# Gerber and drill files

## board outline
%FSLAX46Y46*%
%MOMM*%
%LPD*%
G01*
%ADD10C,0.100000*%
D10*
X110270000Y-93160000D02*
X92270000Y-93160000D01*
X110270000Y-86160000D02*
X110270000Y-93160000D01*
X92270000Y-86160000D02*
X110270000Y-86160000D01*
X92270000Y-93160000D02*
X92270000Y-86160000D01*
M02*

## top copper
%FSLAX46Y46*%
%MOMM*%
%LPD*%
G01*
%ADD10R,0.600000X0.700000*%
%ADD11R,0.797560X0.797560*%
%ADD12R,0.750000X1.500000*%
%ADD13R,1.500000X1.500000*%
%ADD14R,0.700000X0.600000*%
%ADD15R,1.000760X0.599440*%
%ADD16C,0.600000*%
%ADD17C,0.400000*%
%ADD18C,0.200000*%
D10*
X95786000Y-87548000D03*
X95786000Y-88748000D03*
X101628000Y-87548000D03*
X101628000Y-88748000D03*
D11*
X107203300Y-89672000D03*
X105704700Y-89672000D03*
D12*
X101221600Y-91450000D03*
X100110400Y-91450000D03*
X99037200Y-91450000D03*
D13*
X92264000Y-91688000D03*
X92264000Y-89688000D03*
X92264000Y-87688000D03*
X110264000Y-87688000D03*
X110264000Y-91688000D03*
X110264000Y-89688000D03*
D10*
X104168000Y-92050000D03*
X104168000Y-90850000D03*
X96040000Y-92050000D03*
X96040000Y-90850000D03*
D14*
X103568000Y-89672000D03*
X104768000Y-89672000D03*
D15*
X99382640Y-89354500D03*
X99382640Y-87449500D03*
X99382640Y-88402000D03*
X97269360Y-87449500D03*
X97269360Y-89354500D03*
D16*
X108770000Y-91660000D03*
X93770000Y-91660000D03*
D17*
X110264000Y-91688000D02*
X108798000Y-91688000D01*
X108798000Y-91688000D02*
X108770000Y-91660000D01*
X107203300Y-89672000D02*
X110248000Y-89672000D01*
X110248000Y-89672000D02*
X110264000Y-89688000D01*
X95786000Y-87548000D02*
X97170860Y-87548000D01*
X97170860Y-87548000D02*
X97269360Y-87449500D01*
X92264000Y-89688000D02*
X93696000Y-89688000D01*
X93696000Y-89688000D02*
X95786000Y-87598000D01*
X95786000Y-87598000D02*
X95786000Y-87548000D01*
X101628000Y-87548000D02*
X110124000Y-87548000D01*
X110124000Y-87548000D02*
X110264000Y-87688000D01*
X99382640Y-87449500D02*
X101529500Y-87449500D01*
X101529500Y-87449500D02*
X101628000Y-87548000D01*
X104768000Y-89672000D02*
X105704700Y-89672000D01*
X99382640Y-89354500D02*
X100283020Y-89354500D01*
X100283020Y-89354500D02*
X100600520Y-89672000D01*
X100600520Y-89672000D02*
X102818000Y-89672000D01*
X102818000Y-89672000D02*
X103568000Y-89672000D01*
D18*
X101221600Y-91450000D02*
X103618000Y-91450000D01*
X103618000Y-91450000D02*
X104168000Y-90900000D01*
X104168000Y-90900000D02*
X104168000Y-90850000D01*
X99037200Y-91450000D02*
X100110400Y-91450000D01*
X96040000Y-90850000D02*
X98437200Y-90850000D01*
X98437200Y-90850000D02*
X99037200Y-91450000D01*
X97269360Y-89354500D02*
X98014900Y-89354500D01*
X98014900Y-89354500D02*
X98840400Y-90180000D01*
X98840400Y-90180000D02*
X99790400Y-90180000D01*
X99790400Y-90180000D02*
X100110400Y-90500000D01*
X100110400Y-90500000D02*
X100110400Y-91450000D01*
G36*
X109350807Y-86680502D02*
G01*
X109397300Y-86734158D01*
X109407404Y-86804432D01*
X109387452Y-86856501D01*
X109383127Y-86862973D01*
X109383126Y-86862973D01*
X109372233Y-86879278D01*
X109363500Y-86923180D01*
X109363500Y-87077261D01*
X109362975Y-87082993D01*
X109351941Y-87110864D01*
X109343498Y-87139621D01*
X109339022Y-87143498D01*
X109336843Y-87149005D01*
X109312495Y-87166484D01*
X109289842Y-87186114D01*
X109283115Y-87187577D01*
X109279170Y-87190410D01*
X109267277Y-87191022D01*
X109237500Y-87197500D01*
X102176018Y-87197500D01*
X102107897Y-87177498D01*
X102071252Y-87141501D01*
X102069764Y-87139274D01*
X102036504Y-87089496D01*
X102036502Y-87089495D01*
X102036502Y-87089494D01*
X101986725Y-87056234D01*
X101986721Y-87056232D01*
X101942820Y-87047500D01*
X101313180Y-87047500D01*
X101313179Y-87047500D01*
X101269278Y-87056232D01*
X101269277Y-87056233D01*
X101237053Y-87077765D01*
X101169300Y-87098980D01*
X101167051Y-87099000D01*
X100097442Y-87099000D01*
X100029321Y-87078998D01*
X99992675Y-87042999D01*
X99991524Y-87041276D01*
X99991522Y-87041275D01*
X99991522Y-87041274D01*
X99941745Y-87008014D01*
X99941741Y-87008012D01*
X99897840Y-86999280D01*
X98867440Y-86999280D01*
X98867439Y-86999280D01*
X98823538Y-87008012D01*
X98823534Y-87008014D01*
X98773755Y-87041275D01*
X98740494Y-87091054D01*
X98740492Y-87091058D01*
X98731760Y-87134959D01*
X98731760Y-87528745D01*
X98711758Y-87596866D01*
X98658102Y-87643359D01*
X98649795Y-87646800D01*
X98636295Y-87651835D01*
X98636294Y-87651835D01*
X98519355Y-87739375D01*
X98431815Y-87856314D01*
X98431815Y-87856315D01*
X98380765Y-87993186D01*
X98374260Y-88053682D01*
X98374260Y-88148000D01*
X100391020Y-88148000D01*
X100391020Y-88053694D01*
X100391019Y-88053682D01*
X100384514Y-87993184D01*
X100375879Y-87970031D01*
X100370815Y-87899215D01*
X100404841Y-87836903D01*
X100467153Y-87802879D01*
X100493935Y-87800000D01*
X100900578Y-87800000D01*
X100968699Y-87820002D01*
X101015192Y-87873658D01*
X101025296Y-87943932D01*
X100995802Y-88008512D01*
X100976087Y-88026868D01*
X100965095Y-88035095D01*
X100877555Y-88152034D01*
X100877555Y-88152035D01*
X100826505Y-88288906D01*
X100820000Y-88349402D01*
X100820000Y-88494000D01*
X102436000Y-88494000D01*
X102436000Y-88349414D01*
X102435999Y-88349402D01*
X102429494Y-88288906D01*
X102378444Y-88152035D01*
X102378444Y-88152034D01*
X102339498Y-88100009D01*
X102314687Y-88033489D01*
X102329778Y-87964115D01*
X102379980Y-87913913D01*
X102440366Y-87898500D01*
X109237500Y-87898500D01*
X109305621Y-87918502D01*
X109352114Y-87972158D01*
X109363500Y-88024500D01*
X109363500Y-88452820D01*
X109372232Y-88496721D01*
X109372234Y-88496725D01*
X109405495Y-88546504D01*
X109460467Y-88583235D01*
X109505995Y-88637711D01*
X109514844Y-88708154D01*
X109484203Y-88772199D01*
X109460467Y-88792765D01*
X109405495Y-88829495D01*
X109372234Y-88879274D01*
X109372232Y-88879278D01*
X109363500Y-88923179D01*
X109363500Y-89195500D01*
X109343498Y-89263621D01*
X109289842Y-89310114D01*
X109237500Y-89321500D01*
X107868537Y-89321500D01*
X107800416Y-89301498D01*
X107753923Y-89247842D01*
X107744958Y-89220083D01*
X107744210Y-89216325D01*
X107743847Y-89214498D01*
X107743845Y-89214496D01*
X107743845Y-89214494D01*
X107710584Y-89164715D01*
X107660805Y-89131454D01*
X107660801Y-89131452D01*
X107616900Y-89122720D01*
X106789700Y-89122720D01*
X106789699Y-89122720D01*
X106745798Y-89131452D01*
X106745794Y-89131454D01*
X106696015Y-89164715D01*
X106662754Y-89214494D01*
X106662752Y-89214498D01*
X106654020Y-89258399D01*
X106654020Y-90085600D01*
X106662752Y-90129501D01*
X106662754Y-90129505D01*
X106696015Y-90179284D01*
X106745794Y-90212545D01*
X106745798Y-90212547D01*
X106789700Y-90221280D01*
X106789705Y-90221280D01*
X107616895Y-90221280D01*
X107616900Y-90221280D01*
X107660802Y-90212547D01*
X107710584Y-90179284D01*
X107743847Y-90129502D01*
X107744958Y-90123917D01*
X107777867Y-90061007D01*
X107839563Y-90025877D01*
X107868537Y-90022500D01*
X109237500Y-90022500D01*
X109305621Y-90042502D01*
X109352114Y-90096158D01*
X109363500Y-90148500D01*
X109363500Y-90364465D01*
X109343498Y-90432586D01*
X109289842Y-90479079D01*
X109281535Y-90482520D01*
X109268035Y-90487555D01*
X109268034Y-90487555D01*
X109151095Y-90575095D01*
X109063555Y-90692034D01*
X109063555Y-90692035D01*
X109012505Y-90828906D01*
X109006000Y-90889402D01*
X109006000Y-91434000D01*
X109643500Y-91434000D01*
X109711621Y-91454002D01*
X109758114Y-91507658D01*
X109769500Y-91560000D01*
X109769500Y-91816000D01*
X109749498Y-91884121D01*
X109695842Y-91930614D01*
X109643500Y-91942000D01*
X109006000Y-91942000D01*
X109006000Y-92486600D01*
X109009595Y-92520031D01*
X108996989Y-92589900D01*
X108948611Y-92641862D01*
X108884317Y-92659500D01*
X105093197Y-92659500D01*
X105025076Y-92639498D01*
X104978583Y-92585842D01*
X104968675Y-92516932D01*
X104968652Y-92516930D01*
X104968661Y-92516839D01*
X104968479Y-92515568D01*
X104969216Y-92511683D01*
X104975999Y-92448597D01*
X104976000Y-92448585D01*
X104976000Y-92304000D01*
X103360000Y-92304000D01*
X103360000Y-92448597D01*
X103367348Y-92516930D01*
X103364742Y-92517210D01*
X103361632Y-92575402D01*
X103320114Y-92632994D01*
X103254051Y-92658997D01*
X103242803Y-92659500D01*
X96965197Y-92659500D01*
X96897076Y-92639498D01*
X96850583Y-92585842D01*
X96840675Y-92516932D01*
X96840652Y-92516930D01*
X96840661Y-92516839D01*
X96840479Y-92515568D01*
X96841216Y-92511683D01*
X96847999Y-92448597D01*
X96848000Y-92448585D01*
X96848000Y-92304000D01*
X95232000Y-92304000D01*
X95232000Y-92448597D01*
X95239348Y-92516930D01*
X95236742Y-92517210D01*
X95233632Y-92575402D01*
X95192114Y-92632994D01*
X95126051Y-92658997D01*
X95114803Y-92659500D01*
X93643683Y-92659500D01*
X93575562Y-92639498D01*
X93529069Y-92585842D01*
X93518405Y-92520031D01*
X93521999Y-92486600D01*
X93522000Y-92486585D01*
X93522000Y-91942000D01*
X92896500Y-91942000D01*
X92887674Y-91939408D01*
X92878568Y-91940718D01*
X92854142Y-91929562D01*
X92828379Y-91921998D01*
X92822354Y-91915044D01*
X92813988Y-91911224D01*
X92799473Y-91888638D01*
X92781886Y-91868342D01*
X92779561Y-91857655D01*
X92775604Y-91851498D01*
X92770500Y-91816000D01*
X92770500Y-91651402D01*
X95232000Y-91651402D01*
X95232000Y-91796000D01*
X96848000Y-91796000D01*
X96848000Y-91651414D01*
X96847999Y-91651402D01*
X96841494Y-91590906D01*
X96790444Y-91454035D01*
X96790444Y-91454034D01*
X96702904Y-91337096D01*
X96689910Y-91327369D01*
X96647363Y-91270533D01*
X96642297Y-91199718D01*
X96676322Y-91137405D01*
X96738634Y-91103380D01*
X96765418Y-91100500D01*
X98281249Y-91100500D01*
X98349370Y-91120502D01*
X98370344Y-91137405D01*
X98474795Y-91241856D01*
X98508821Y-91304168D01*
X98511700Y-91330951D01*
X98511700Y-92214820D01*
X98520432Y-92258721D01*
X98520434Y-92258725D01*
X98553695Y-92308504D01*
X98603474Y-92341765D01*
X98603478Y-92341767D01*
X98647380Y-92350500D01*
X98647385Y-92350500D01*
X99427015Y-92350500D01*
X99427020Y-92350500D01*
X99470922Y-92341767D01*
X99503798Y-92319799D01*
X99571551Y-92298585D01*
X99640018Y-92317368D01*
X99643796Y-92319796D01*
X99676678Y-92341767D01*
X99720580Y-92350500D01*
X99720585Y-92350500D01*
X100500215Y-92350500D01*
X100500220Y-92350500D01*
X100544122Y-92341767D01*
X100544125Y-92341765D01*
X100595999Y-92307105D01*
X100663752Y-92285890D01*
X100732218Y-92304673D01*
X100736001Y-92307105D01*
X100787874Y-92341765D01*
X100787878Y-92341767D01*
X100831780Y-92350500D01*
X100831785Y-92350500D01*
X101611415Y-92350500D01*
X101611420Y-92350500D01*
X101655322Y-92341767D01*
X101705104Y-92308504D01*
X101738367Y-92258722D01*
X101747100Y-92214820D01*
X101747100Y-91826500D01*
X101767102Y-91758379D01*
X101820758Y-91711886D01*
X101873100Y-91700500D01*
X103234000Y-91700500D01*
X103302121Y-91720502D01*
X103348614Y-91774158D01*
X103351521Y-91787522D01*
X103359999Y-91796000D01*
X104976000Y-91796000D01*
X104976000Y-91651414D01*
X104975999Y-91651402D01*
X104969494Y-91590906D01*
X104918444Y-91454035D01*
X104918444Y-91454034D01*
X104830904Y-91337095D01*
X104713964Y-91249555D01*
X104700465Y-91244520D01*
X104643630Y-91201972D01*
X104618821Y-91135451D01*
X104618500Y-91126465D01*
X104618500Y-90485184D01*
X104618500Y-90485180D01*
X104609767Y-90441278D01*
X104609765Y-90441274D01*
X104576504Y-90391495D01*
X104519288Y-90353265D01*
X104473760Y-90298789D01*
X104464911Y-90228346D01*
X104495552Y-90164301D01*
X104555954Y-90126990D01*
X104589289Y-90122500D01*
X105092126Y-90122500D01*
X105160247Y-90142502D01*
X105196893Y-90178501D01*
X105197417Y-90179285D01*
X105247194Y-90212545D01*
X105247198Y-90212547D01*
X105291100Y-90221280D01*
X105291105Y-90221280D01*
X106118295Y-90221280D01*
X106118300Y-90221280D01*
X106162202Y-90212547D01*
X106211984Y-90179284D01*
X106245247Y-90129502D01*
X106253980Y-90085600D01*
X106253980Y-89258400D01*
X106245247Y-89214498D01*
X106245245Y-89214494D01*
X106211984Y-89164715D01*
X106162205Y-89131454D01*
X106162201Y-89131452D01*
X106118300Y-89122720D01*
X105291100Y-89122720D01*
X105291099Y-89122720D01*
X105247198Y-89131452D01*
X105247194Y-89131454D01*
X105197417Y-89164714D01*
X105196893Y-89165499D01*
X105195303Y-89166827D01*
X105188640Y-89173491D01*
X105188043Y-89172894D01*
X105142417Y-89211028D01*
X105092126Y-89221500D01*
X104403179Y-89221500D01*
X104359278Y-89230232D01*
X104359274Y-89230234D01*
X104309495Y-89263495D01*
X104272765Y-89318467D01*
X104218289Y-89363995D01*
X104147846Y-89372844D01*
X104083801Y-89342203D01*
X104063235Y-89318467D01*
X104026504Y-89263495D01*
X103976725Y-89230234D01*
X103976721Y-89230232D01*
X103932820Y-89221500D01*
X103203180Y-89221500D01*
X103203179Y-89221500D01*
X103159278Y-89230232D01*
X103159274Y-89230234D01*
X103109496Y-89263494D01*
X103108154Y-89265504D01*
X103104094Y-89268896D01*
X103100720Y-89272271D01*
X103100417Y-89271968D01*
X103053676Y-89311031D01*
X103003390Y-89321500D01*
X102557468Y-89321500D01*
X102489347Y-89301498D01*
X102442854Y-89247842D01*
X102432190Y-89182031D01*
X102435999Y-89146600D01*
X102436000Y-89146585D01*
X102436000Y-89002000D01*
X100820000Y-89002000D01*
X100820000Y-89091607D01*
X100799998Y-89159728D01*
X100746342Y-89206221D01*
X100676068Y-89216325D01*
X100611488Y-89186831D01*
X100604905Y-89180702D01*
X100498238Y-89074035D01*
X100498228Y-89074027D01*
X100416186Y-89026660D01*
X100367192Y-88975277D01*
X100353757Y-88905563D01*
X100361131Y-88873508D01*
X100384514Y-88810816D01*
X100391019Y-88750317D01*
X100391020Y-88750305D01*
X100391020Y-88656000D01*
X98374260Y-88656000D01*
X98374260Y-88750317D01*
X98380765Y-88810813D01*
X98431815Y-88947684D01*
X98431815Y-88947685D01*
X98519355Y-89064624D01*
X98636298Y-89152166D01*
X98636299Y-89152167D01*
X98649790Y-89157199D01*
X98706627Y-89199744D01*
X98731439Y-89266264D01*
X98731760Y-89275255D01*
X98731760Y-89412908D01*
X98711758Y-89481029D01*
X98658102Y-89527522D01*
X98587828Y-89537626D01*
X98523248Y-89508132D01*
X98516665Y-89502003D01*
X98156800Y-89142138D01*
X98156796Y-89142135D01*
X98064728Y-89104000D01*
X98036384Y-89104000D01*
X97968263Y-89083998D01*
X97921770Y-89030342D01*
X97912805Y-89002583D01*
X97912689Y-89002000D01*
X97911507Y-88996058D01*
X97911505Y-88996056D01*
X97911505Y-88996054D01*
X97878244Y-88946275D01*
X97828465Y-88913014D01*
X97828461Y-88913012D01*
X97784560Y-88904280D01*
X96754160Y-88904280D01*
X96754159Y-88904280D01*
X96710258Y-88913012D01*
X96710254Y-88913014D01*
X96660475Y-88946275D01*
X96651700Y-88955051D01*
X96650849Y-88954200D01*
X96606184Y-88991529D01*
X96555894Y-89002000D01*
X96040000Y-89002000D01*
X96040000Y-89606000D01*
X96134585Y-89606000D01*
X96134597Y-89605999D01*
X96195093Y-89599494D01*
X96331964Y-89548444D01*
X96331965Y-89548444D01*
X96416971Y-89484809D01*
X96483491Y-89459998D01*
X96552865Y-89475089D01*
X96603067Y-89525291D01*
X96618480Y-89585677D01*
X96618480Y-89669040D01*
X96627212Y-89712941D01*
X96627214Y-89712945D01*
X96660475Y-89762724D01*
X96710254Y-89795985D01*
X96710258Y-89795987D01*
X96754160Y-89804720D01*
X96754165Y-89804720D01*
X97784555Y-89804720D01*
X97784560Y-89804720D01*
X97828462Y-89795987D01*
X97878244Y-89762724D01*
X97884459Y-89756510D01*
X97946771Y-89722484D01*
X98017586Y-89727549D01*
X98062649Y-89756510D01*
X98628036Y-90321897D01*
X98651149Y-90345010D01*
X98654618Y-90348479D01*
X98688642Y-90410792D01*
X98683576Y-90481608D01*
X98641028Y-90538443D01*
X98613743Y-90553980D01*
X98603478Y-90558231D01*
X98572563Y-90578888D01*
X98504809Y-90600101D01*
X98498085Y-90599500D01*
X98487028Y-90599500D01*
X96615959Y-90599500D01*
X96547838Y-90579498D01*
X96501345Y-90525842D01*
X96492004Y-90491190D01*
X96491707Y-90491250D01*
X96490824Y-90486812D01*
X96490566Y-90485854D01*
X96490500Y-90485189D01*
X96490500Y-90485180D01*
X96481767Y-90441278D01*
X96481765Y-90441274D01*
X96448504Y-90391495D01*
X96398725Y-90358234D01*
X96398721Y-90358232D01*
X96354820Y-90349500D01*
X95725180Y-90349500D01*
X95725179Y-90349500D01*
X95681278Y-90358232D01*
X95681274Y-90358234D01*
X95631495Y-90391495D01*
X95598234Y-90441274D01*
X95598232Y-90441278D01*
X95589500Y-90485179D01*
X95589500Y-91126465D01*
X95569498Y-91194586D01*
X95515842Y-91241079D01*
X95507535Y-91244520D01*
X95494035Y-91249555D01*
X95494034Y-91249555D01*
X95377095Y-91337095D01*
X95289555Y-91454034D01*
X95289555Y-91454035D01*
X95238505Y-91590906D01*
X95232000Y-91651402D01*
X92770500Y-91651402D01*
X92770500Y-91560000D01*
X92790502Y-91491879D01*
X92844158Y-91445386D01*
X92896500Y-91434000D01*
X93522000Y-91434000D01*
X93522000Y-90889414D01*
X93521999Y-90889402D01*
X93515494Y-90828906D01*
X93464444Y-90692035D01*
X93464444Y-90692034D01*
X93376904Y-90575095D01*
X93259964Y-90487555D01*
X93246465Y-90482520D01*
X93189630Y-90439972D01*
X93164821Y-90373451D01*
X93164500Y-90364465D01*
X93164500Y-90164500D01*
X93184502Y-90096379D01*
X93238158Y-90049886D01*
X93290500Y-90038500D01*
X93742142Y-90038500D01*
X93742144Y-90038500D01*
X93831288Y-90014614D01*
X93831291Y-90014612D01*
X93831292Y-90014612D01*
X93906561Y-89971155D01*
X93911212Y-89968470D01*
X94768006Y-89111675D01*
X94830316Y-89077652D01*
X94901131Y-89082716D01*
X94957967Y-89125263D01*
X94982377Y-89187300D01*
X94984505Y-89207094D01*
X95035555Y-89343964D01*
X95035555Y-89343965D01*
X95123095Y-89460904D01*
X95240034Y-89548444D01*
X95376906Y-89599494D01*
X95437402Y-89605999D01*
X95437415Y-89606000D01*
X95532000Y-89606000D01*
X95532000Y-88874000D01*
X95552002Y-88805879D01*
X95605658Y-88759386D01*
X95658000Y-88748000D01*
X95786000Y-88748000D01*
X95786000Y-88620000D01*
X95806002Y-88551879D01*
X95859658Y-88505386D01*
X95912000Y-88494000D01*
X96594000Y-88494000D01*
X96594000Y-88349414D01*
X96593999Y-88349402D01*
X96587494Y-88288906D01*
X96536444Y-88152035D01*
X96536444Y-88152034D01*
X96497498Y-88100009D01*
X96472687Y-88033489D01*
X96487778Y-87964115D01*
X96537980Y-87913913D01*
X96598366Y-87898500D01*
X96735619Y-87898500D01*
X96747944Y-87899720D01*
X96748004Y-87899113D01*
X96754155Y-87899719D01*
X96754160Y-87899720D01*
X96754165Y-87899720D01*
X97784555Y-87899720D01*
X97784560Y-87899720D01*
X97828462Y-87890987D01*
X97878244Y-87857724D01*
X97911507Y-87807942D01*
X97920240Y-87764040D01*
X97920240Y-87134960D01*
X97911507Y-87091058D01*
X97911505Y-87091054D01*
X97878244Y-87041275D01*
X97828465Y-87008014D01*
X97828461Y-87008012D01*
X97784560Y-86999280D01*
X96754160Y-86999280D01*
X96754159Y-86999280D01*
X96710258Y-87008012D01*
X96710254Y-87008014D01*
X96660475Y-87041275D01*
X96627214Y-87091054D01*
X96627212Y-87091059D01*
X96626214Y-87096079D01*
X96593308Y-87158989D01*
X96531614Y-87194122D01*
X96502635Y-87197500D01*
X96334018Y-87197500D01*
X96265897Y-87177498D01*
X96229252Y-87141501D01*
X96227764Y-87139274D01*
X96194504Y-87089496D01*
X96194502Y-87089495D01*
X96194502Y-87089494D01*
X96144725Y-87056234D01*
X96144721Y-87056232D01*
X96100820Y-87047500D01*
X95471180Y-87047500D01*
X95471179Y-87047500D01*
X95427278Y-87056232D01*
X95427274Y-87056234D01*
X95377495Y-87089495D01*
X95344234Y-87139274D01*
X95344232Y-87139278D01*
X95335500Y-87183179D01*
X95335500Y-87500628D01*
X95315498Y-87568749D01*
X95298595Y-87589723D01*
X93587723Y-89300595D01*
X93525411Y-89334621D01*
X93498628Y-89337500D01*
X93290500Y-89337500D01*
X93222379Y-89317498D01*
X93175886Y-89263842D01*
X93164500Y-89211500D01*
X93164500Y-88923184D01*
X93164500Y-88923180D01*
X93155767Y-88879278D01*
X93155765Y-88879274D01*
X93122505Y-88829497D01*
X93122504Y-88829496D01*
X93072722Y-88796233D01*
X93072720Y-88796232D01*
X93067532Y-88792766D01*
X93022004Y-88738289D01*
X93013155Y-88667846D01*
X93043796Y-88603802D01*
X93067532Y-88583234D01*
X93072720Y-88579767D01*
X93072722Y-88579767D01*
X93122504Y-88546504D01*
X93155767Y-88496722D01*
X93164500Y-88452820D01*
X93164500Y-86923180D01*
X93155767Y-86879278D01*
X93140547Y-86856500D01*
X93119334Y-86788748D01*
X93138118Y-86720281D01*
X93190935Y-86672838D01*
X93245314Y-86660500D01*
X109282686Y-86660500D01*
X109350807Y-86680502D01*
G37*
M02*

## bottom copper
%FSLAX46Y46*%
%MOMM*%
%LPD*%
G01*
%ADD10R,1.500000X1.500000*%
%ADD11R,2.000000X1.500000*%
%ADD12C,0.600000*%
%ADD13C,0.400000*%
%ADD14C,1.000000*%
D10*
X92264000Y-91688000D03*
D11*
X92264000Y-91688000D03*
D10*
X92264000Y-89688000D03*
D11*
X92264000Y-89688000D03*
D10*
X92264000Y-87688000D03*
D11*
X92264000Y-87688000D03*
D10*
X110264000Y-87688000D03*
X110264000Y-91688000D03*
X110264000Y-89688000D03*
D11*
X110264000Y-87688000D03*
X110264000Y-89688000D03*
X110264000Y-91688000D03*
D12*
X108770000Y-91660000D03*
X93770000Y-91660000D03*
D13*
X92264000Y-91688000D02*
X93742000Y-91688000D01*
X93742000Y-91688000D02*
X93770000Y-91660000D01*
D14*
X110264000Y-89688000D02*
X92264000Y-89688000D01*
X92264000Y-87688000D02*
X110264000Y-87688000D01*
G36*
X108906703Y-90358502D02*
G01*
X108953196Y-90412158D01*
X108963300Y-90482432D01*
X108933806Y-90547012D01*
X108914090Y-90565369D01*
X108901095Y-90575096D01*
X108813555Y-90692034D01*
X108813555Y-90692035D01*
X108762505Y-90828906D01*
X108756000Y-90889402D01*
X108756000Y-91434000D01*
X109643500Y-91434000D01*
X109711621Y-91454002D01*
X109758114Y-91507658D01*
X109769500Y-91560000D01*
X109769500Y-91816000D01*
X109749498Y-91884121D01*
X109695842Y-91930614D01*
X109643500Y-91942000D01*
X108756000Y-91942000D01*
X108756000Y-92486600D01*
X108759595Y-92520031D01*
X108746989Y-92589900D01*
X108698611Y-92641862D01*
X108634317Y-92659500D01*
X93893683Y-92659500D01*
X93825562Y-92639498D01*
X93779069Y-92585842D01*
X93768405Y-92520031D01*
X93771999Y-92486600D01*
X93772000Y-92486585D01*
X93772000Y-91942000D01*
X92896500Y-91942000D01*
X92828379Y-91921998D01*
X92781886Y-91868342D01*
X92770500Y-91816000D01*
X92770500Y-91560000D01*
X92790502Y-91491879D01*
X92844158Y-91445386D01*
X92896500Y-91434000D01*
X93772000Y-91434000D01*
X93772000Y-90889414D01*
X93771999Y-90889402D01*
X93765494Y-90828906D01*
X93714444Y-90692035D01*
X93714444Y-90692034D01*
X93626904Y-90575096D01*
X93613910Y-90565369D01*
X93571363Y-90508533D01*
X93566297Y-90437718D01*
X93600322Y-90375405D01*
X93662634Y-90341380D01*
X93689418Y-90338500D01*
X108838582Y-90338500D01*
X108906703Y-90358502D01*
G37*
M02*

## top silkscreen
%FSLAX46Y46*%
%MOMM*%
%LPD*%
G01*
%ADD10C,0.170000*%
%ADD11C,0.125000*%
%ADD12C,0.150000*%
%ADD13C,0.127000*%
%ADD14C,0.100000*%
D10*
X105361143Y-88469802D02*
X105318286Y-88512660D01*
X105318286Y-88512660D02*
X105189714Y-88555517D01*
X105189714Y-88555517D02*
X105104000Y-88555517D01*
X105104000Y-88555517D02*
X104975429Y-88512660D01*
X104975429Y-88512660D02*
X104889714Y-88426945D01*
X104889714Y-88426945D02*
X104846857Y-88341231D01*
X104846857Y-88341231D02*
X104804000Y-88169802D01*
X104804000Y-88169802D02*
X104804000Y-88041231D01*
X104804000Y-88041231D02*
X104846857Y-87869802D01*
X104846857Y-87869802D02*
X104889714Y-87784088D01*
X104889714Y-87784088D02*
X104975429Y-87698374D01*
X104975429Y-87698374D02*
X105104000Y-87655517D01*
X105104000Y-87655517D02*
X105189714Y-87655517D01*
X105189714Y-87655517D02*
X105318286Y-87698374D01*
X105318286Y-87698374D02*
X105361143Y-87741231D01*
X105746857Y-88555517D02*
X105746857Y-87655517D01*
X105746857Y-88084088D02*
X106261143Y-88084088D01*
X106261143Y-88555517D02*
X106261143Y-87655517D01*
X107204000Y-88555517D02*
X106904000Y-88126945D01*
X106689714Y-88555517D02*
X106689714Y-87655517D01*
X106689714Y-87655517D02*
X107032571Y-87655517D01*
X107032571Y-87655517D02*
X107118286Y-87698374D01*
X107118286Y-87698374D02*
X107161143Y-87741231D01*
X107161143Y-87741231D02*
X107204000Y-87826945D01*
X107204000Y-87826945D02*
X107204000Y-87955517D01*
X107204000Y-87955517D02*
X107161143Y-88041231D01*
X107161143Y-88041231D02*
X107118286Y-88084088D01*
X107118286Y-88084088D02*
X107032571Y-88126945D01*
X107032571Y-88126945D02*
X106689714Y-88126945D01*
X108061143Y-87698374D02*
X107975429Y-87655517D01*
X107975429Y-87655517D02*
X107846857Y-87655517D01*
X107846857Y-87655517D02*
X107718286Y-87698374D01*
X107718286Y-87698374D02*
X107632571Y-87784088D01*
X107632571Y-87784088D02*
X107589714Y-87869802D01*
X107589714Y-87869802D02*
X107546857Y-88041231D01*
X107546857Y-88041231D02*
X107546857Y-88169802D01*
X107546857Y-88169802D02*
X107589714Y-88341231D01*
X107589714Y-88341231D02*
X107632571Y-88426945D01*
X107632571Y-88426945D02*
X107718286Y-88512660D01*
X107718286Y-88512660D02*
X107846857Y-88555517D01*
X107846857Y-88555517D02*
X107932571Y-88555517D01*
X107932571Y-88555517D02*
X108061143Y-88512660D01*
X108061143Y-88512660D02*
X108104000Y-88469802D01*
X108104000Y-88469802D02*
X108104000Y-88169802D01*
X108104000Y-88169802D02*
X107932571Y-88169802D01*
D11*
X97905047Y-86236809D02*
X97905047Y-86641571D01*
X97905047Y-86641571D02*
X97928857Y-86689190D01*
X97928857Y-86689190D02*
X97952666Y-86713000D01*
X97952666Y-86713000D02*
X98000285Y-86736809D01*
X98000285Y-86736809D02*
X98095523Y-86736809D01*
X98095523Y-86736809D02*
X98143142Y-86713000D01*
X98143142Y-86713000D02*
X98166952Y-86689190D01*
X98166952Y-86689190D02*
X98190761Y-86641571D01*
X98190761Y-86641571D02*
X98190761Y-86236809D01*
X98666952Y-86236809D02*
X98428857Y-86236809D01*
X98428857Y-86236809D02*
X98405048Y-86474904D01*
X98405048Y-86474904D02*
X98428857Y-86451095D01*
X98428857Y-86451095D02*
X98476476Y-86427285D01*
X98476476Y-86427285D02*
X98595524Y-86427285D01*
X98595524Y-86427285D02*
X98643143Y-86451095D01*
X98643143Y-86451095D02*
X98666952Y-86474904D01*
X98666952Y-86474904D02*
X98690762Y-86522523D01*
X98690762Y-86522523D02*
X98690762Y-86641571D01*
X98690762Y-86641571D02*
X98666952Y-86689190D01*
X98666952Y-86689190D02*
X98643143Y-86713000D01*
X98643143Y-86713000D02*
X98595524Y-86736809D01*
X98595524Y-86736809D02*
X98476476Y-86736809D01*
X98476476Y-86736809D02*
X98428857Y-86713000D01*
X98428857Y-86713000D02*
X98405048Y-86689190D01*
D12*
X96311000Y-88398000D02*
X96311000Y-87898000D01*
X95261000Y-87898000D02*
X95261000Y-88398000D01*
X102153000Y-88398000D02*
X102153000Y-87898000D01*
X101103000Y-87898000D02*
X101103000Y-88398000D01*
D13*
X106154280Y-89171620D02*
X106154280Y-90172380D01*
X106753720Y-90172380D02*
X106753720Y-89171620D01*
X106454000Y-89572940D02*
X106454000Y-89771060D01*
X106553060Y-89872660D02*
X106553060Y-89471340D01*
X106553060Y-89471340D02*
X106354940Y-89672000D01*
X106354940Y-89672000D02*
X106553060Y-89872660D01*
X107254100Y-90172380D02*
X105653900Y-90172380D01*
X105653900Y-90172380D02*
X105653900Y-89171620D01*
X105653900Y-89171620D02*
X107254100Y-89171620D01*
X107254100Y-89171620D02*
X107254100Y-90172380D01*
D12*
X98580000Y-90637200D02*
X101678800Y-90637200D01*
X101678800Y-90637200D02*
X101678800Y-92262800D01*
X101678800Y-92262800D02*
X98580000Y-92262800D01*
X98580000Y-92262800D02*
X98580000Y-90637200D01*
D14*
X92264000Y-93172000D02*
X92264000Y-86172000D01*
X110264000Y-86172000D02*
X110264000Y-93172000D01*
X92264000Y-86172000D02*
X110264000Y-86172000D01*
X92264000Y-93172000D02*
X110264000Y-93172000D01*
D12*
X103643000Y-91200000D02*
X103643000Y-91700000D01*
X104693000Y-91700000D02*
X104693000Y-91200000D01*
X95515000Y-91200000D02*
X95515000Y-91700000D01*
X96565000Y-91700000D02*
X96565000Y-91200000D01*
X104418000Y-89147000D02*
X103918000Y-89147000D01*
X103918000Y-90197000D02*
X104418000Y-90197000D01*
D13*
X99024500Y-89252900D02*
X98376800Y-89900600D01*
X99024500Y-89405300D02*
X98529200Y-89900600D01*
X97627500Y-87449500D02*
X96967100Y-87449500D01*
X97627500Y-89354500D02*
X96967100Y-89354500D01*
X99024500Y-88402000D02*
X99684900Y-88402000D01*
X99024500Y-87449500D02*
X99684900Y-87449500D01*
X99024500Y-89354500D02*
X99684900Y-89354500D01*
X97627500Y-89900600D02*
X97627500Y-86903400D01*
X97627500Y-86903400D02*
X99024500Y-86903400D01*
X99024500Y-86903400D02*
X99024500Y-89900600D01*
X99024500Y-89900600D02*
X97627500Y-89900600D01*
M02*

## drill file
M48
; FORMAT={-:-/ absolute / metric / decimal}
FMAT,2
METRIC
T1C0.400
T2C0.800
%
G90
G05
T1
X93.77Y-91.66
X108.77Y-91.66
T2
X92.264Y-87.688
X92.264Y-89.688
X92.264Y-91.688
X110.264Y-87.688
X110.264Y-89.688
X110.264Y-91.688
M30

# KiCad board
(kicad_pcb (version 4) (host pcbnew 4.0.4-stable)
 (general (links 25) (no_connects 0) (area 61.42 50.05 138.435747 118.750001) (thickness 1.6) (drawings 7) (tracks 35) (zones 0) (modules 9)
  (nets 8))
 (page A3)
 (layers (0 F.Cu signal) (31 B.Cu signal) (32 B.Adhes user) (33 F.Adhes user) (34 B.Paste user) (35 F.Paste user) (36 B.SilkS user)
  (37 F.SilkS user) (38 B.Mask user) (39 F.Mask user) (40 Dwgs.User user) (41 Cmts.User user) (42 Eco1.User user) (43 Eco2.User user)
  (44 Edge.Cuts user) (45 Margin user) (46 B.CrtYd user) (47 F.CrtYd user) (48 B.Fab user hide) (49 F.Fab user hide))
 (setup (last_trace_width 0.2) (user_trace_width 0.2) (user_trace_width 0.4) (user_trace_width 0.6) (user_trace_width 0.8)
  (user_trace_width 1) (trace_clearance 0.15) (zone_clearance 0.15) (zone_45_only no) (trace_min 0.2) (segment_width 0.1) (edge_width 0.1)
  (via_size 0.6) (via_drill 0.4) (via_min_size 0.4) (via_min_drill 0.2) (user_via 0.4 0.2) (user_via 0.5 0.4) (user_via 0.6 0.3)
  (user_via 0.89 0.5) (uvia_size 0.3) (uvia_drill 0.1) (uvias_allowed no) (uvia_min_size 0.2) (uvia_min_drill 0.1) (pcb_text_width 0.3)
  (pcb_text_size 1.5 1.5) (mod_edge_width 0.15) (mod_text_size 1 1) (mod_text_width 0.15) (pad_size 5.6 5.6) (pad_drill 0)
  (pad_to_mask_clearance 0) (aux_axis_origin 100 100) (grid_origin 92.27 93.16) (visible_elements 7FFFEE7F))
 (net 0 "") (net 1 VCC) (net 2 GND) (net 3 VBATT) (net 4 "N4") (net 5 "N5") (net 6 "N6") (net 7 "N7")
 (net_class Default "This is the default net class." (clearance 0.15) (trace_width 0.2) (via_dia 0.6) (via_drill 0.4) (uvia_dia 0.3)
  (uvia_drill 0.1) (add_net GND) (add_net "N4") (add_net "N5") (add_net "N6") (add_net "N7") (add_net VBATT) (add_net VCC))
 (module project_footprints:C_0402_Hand (layer F.Cu) (at 95.786 88.148 270)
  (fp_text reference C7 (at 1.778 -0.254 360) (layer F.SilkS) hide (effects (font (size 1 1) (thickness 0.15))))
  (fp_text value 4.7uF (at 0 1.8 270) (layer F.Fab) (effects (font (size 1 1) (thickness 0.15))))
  (fp_line (start 0.25 -0.525) (end -0.25 -0.525) (layer F.SilkS) (width 0.15))
  (fp_line (start -0.25 0.525) (end 0.25 0.525) (layer F.SilkS) (width 0.15))
  (pad 1 smd rect (at -0.6 0 270) (size 0.7 0.6) (layers F.Cu F.Paste F.Mask) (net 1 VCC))
  (pad 2 smd rect (at 0.6 0 270) (size 0.7 0.6) (layers F.Cu F.Paste F.Mask) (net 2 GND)))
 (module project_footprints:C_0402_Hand (layer F.Cu) (at 101.628 88.148 270)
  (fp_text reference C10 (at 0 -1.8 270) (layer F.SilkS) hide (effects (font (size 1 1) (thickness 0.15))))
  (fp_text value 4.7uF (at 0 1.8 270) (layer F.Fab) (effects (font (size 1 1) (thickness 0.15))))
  (fp_line (start 0.25 -0.525) (end -0.25 -0.525) (layer F.SilkS) (width 0.15))
  (fp_line (start -0.25 0.525) (end 0.25 0.525) (layer F.SilkS) (width 0.15))
  (pad 1 smd rect (at -0.6 0 270) (size 0.7 0.6) (layers F.Cu F.Paste F.Mask) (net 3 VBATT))
  (pad 2 smd rect (at 0.6 0 270) (size 0.7 0.6) (layers F.Cu F.Paste F.Mask) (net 2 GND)))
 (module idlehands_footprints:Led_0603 (layer F.Cu) (at 106.454 89.672 180)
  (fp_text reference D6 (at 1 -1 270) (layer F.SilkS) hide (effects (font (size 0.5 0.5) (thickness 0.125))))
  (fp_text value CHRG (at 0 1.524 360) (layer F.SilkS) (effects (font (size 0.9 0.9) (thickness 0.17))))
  (fp_line (start 0.29972 0.50038) (end 0.29972 -0.50038) (layer F.SilkS) (width 0.127))
  (fp_line (start -0.29972 -0.50038) (end -0.29972 0.50038) (layer F.SilkS) (width 0.127))
  (fp_line (start 0 0.09906) (end 0 -0.09906) (layer F.SilkS) (width 0.127))
  (fp_line (start -0.09906 -0.20066) (end -0.09906 0.20066) (layer F.SilkS) (width 0.127))
  (fp_line (start -0.09906 0.20066) (end 0.09906 0) (layer F.SilkS) (width 0.127))
  (fp_line (start 0.09906 0) (end -0.09906 -0.20066) (layer F.SilkS) (width 0.127))
  (fp_line (start -0.8001 -0.50038) (end 0.8001 -0.50038) (layer F.SilkS) (width 0.127))
  (fp_line (start 0.8001 -0.50038) (end 0.8001 0.50038) (layer F.SilkS) (width 0.127))
  (fp_line (start 0.8001 0.50038) (end -0.8001 0.50038) (layer F.SilkS) (width 0.127))
  (fp_line (start -0.8001 0.50038) (end -0.8001 -0.50038) (layer F.SilkS) (width 0.127))
  (pad 2 smd rect (at -0.7493 0 180) (size 0.79756 0.79756) (layers F.Cu F.Paste F.Mask) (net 1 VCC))
  (pad 1 smd rect (at 0.7493 0 180) (size 0.79756 0.79756) (layers F.Cu F.Paste F.Mask) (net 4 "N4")))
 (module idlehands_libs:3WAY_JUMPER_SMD (layer F.Cu) (at 100.104 91.45)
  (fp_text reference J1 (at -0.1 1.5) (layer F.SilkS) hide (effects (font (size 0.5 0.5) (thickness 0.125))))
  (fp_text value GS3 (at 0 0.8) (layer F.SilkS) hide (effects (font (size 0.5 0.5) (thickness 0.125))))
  (fp_line (start -1.524 -0.8128) (end 1.5748 -0.8128) (layer F.SilkS) (width 0.15))
  (fp_line (start 1.5748 -0.8128) (end 1.5748 0.8128) (layer F.SilkS) (width 0.15))
  (fp_line (start 1.5748 0.8128) (end -1.524 0.8128) (layer F.SilkS) (width 0.15))
  (fp_line (start -1.524 0.8128) (end -1.524 -0.8128) (layer F.SilkS) (width 0.15))
  (pad 1 smd rect (at 1.1176 0) (size 0.75 1.5) (layers F.Cu F.Paste F.Mask) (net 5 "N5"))
  (pad 2 smd rect (at 0.0064 0) (size 0.75 1.5) (layers F.Cu F.Paste F.Mask) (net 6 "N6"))
  (pad 3 smd rect (at -1.0668 0) (size 0.75 1.5) (layers F.Cu F.Paste F.Mask) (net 6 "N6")))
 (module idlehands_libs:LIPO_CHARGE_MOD (layer F.Cu) (at 101.264 89.672)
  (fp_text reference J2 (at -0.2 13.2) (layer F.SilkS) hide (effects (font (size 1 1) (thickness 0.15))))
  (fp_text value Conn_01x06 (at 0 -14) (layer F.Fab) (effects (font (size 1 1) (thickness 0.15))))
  (fp_line (start -9 3.5) (end -9 -3.5) (layer F.SilkS) (width 0.1))
  (fp_line (start 9 -3.5) (end 9 3.5) (layer F.SilkS) (width 0.1))
  (fp_line (start -9 -3.5) (end 9 -3.5) (layer F.SilkS) (width 0.1))
  (fp_line (start -9 3.5) (end 9 3.5) (layer F.SilkS) (width 0.1))
  (pad 3 thru_hole rect (at -9 2.016) (size 1.5 1.5) (drill 0.8) (layers *.Cu *.Mask) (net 2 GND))
  (pad 3 smd rect (at -9 2.016) (size 2 1.5) (layers B.Cu B.Mask) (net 2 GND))
  (pad 2 thru_hole rect (at -9 0.016) (size 1.5 1.5) (drill 0.8) (layers *.Cu *.Mask) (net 1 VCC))
  (pad 2 smd rect (at -9 0.016) (size 2 1.5) (layers B.Cu B.Mask) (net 1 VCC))
  (pad 1 thru_hole rect (at -9 -1.984) (size 1.5 1.5) (drill 0.8) (layers *.Cu *.Mask) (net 3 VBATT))
  (pad 1 smd rect (at -9 -1.984) (size 2 1.5) (layers B.Cu B.Mask) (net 3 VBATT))
  (pad 4 thru_hole rect (at 9 -1.984) (size 1.5 1.5) (drill 0.8) (layers *.Cu *.Mask) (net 3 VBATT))
  (pad 6 thru_hole rect (at 9 2.016) (size 1.5 1.5) (drill 0.8) (layers *.Cu *.Mask) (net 2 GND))
  (pad 5 thru_hole rect (at 9 0.016) (size 1.5 1.5) (drill 0.8) (layers *.Cu *.Mask) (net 1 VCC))
  (pad 4 smd rect (at 9 -1.984) (size 2 1.5) (layers B.Cu B.Mask) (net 3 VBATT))
  (pad 5 smd rect (at 9 0.016) (size 2 1.5) (layers B.Cu B.Mask) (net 1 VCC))
  (pad 6 smd rect (at 9 2.016) (size 2 1.5) (layers B.Cu B.Mask) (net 2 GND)))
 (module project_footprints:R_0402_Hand (layer F.Cu) (at 104.168 91.45 90)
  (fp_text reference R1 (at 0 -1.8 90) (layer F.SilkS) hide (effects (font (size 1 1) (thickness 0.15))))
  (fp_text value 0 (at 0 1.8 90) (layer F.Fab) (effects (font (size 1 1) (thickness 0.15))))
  (fp_line (start 0.25 -0.525) (end -0.25 -0.525) (layer F.SilkS) (width 0.15))
  (fp_line (start -0.25 0.525) (end 0.25 0.525) (layer F.SilkS) (width 0.15))
  (pad 1 smd rect (at -0.6 0 90) (size 0.7 0.6) (layers F.Cu F.Paste F.Mask) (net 2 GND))
  (pad 2 smd rect (at 0.6 0 90) (size 0.7 0.6) (layers F.Cu F.Paste F.Mask) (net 5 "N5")))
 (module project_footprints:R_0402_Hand (layer F.Cu) (at 96.04 91.45 90)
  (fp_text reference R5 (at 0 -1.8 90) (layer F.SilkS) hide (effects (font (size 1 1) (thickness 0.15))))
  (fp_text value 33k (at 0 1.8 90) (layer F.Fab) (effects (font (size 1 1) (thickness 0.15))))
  (fp_line (start 0.25 -0.525) (end -0.25 -0.525) (layer F.SilkS) (width 0.15))
  (fp_line (start -0.25 0.525) (end 0.25 0.525) (layer F.SilkS) (width 0.15))
  (pad 1 smd rect (at -0.6 0 90) (size 0.7 0.6) (layers F.Cu F.Paste F.Mask) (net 2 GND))
  (pad 2 smd rect (at 0.6 0 90) (size 0.7 0.6) (layers F.Cu F.Paste F.Mask) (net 6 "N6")))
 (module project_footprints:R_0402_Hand (layer F.Cu) (at 104.168 89.672)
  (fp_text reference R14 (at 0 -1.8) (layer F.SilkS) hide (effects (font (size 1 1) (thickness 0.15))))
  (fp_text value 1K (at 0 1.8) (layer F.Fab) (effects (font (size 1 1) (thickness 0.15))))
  (fp_line (start 0.25 -0.525) (end -0.25 -0.525) (layer F.SilkS) (width 0.15))
  (fp_line (start -0.25 0.525) (end 0.25 0.525) (layer F.SilkS) (width 0.15))
  (pad 1 smd rect (at -0.6 0) (size 0.7 0.6) (layers F.Cu F.Paste F.Mask) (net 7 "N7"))
  (pad 2 smd rect (at 0.6 0) (size 0.7 0.6) (layers F.Cu F.Paste F.Mask) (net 4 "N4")))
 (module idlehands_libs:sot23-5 (layer F.Cu) (at 98.326 88.402 90)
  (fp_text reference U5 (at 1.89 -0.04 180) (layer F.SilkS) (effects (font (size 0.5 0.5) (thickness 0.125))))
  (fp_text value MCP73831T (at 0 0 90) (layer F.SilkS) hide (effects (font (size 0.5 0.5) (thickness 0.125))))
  (fp_line (start -0.8509 0.6985) (end -1.4986 0.0508) (layer F.SilkS) (width 0.127))
  (fp_line (start -1.0033 0.6985) (end -1.4986 0.2032) (layer F.SilkS) (width 0.127))
  (fp_line (start 0.9525 -0.6985) (end 0.9525 -1.3589) (layer F.SilkS) (width 0.127))
  (fp_line (start -0.9525 -0.6985) (end -0.9525 -1.3589) (layer F.SilkS) (width 0.127))
  (fp_line (start 0 0.6985) (end 0 1.3589) (layer F.SilkS) (width 0.127))
  (fp_line (start 0.9525 0.6985) (end 0.9525 1.3589) (layer F.SilkS) (width 0.127))
  (fp_line (start -0.9525 0.6985) (end -0.9525 1.3589) (layer F.SilkS) (width 0.127))
  (fp_line (start -1.4986 -0.6985) (end 1.4986 -0.6985) (layer F.SilkS) (width 0.127))
  (fp_line (start 1.4986 -0.6985) (end 1.4986 0.6985) (layer F.SilkS) (width 0.127))
  (fp_line (start 1.4986 0.6985) (end -1.4986 0.6985) (layer F.SilkS) (width 0.127))
  (fp_line (start -1.4986 0.6985) (end -1.4986 -0.6985) (layer F.SilkS) (width 0.127))
  (pad 1 smd rect (at -0.9525 1.05664 90) (size 0.59944 1.00076) (layers F.Cu F.Paste F.Mask) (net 7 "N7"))
  (pad 3 smd rect (at 0.9525 1.05664 90) (size 0.59944 1.00076) (layers F.Cu F.Paste F.Mask) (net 3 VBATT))
  (pad 2 smd rect (at 0 1.05664 90) (size 0.59944 1.00076) (layers F.Cu F.Paste F.Mask) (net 2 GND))
  (pad 4 smd rect (at 0.9525 -1.05664 90) (size 0.59944 1.00076) (layers F.Cu F.Paste F.Mask) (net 1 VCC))
  (pad 5 smd rect (at -0.9525 -1.05664 90) (size 0.59944 1.00076) (layers F.Cu F.Paste F.Mask) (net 6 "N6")))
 (gr_line (start 110.27 93.16) (end 92.27 93.16) (layer Edge.Cuts) (width 0.1))
 (gr_line (start 110.27 86.16) (end 110.27 93.16) (layer Edge.Cuts) (width 0.1))
 (gr_line (start 92.27 86.16) (end 110.27 86.16) (layer Edge.Cuts) (width 0.1))
 (gr_line (start 92.27 93.16) (end 92.27 86.16) (layer Edge.Cuts) (width 0.1))
 (segment (start 110.264 91.688) (end 108.798 91.688) (width 0.4) (layer F.Cu) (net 2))
 (segment (start 108.798 91.688) (end 108.77 91.66) (width 0.4) (layer F.Cu) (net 2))
 (via (at 108.77 91.66) (size 0.6) (drill 0.4) (layers F.Cu B.Cu) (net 2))
 (segment (start 92.264 91.688) (end 93.742 91.688) (width 0.4) (layer B.Cu) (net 2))
 (segment (start 93.742 91.688) (end 93.77 91.66) (width 0.4) (layer B.Cu) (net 2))
 (via (at 93.77 91.66) (size 0.6) (drill 0.4) (layers F.Cu B.Cu) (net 2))
 (segment (start 110.264 89.688) (end 92.264 89.688) (width 1) (layer B.Cu) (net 1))
 (segment (start 107.2033 89.672) (end 110.248 89.672) (width 0.4) (layer F.Cu) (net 1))
 (segment (start 110.248 89.672) (end 110.264 89.688) (width 0.4) (layer F.Cu) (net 1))
 (segment (start 95.786 87.548) (end 97.17086 87.548) (width 0.4) (layer F.Cu) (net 1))
 (segment (start 97.17086 87.548) (end 97.26936 87.4495) (width 0.4) (layer F.Cu) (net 1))
 (segment (start 92.264 89.688) (end 93.696 89.688) (width 0.4) (layer F.Cu) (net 1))
 (segment (start 93.696 89.688) (end 95.786 87.598) (width 0.4) (layer F.Cu) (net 1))
 (segment (start 95.786 87.598) (end 95.786 87.548) (width 0.4) (layer F.Cu) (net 1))
 (segment (start 92.264 87.688) (end 110.264 87.688) (width 1) (layer B.Cu) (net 3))
 (segment (start 101.628 87.548) (end 110.124 87.548) (width 0.4) (layer F.Cu) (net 3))
 (segment (start 110.124 87.548) (end 110.264 87.688) (width 0.4) (layer F.Cu) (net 3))
 (segment (start 99.38264 87.4495) (end 101.5295 87.4495) (width 0.4) (layer F.Cu) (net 3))
 (segment (start 101.5295 87.4495) (end 101.628 87.548) (width 0.4) (layer F.Cu) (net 3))
 (segment (start 104.768 89.672) (end 105.7047 89.672) (width 0.4) (layer F.Cu) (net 4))
 (segment (start 99.38264 89.3545) (end 100.28302 89.3545) (width 0.4) (layer F.Cu) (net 7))
 (segment (start 100.28302 89.3545) (end 100.60052 89.672) (width 0.4) (layer F.Cu) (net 7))
 (segment (start 100.60052 89.672) (end 102.818 89.672) (width 0.4) (layer F.Cu) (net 7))
 (segment (start 102.818 89.672) (end 103.568 89.672) (width 0.4) (layer F.Cu) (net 7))
 (segment (start 101.2216 91.45) (end 103.618 91.45) (width 0.2) (layer F.Cu) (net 5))
 (segment (start 103.618 91.45) (end 104.168 90.9) (width 0.2) (layer F.Cu) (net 5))
 (segment (start 104.168 90.9) (end 104.168 90.85) (width 0.2) (layer F.Cu) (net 5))
 (segment (start 99.0372 91.45) (end 100.1104 91.45) (width 0.2) (layer F.Cu) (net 6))
 (segment (start 96.04 90.85) (end 98.4372 90.85) (width 0.2) (layer F.Cu) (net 6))
 (segment (start 98.4372 90.85) (end 99.0372 91.45) (width 0.2) (layer F.Cu) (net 6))
 (segment (start 97.26936 89.3545) (end 98.0149 89.3545) (width 0.2) (layer F.Cu) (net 6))
 (segment (start 98.0149 89.3545) (end 98.8404 90.18) (width 0.2) (layer F.Cu) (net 6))
 (segment (start 98.8404 90.18) (end 99.7904 90.18) (width 0.2) (layer F.Cu) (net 6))
 (segment (start 99.7904 90.18) (end 100.1104 90.5) (width 0.2) (layer F.Cu) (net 6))
 (segment (start 100.1104 90.5) (end 100.1104 91.45) (width 0.2) (layer F.Cu) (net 6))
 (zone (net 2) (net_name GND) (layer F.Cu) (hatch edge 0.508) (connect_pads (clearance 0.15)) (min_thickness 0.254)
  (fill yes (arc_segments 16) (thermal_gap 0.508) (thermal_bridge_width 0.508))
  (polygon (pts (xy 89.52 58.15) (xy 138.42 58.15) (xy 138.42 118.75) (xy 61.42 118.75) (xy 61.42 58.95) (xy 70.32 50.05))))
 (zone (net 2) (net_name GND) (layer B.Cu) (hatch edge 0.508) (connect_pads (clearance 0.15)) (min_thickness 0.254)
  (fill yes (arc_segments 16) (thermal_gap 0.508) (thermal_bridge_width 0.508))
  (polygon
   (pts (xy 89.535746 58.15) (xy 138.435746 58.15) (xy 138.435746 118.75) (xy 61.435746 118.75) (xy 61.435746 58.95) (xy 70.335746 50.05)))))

